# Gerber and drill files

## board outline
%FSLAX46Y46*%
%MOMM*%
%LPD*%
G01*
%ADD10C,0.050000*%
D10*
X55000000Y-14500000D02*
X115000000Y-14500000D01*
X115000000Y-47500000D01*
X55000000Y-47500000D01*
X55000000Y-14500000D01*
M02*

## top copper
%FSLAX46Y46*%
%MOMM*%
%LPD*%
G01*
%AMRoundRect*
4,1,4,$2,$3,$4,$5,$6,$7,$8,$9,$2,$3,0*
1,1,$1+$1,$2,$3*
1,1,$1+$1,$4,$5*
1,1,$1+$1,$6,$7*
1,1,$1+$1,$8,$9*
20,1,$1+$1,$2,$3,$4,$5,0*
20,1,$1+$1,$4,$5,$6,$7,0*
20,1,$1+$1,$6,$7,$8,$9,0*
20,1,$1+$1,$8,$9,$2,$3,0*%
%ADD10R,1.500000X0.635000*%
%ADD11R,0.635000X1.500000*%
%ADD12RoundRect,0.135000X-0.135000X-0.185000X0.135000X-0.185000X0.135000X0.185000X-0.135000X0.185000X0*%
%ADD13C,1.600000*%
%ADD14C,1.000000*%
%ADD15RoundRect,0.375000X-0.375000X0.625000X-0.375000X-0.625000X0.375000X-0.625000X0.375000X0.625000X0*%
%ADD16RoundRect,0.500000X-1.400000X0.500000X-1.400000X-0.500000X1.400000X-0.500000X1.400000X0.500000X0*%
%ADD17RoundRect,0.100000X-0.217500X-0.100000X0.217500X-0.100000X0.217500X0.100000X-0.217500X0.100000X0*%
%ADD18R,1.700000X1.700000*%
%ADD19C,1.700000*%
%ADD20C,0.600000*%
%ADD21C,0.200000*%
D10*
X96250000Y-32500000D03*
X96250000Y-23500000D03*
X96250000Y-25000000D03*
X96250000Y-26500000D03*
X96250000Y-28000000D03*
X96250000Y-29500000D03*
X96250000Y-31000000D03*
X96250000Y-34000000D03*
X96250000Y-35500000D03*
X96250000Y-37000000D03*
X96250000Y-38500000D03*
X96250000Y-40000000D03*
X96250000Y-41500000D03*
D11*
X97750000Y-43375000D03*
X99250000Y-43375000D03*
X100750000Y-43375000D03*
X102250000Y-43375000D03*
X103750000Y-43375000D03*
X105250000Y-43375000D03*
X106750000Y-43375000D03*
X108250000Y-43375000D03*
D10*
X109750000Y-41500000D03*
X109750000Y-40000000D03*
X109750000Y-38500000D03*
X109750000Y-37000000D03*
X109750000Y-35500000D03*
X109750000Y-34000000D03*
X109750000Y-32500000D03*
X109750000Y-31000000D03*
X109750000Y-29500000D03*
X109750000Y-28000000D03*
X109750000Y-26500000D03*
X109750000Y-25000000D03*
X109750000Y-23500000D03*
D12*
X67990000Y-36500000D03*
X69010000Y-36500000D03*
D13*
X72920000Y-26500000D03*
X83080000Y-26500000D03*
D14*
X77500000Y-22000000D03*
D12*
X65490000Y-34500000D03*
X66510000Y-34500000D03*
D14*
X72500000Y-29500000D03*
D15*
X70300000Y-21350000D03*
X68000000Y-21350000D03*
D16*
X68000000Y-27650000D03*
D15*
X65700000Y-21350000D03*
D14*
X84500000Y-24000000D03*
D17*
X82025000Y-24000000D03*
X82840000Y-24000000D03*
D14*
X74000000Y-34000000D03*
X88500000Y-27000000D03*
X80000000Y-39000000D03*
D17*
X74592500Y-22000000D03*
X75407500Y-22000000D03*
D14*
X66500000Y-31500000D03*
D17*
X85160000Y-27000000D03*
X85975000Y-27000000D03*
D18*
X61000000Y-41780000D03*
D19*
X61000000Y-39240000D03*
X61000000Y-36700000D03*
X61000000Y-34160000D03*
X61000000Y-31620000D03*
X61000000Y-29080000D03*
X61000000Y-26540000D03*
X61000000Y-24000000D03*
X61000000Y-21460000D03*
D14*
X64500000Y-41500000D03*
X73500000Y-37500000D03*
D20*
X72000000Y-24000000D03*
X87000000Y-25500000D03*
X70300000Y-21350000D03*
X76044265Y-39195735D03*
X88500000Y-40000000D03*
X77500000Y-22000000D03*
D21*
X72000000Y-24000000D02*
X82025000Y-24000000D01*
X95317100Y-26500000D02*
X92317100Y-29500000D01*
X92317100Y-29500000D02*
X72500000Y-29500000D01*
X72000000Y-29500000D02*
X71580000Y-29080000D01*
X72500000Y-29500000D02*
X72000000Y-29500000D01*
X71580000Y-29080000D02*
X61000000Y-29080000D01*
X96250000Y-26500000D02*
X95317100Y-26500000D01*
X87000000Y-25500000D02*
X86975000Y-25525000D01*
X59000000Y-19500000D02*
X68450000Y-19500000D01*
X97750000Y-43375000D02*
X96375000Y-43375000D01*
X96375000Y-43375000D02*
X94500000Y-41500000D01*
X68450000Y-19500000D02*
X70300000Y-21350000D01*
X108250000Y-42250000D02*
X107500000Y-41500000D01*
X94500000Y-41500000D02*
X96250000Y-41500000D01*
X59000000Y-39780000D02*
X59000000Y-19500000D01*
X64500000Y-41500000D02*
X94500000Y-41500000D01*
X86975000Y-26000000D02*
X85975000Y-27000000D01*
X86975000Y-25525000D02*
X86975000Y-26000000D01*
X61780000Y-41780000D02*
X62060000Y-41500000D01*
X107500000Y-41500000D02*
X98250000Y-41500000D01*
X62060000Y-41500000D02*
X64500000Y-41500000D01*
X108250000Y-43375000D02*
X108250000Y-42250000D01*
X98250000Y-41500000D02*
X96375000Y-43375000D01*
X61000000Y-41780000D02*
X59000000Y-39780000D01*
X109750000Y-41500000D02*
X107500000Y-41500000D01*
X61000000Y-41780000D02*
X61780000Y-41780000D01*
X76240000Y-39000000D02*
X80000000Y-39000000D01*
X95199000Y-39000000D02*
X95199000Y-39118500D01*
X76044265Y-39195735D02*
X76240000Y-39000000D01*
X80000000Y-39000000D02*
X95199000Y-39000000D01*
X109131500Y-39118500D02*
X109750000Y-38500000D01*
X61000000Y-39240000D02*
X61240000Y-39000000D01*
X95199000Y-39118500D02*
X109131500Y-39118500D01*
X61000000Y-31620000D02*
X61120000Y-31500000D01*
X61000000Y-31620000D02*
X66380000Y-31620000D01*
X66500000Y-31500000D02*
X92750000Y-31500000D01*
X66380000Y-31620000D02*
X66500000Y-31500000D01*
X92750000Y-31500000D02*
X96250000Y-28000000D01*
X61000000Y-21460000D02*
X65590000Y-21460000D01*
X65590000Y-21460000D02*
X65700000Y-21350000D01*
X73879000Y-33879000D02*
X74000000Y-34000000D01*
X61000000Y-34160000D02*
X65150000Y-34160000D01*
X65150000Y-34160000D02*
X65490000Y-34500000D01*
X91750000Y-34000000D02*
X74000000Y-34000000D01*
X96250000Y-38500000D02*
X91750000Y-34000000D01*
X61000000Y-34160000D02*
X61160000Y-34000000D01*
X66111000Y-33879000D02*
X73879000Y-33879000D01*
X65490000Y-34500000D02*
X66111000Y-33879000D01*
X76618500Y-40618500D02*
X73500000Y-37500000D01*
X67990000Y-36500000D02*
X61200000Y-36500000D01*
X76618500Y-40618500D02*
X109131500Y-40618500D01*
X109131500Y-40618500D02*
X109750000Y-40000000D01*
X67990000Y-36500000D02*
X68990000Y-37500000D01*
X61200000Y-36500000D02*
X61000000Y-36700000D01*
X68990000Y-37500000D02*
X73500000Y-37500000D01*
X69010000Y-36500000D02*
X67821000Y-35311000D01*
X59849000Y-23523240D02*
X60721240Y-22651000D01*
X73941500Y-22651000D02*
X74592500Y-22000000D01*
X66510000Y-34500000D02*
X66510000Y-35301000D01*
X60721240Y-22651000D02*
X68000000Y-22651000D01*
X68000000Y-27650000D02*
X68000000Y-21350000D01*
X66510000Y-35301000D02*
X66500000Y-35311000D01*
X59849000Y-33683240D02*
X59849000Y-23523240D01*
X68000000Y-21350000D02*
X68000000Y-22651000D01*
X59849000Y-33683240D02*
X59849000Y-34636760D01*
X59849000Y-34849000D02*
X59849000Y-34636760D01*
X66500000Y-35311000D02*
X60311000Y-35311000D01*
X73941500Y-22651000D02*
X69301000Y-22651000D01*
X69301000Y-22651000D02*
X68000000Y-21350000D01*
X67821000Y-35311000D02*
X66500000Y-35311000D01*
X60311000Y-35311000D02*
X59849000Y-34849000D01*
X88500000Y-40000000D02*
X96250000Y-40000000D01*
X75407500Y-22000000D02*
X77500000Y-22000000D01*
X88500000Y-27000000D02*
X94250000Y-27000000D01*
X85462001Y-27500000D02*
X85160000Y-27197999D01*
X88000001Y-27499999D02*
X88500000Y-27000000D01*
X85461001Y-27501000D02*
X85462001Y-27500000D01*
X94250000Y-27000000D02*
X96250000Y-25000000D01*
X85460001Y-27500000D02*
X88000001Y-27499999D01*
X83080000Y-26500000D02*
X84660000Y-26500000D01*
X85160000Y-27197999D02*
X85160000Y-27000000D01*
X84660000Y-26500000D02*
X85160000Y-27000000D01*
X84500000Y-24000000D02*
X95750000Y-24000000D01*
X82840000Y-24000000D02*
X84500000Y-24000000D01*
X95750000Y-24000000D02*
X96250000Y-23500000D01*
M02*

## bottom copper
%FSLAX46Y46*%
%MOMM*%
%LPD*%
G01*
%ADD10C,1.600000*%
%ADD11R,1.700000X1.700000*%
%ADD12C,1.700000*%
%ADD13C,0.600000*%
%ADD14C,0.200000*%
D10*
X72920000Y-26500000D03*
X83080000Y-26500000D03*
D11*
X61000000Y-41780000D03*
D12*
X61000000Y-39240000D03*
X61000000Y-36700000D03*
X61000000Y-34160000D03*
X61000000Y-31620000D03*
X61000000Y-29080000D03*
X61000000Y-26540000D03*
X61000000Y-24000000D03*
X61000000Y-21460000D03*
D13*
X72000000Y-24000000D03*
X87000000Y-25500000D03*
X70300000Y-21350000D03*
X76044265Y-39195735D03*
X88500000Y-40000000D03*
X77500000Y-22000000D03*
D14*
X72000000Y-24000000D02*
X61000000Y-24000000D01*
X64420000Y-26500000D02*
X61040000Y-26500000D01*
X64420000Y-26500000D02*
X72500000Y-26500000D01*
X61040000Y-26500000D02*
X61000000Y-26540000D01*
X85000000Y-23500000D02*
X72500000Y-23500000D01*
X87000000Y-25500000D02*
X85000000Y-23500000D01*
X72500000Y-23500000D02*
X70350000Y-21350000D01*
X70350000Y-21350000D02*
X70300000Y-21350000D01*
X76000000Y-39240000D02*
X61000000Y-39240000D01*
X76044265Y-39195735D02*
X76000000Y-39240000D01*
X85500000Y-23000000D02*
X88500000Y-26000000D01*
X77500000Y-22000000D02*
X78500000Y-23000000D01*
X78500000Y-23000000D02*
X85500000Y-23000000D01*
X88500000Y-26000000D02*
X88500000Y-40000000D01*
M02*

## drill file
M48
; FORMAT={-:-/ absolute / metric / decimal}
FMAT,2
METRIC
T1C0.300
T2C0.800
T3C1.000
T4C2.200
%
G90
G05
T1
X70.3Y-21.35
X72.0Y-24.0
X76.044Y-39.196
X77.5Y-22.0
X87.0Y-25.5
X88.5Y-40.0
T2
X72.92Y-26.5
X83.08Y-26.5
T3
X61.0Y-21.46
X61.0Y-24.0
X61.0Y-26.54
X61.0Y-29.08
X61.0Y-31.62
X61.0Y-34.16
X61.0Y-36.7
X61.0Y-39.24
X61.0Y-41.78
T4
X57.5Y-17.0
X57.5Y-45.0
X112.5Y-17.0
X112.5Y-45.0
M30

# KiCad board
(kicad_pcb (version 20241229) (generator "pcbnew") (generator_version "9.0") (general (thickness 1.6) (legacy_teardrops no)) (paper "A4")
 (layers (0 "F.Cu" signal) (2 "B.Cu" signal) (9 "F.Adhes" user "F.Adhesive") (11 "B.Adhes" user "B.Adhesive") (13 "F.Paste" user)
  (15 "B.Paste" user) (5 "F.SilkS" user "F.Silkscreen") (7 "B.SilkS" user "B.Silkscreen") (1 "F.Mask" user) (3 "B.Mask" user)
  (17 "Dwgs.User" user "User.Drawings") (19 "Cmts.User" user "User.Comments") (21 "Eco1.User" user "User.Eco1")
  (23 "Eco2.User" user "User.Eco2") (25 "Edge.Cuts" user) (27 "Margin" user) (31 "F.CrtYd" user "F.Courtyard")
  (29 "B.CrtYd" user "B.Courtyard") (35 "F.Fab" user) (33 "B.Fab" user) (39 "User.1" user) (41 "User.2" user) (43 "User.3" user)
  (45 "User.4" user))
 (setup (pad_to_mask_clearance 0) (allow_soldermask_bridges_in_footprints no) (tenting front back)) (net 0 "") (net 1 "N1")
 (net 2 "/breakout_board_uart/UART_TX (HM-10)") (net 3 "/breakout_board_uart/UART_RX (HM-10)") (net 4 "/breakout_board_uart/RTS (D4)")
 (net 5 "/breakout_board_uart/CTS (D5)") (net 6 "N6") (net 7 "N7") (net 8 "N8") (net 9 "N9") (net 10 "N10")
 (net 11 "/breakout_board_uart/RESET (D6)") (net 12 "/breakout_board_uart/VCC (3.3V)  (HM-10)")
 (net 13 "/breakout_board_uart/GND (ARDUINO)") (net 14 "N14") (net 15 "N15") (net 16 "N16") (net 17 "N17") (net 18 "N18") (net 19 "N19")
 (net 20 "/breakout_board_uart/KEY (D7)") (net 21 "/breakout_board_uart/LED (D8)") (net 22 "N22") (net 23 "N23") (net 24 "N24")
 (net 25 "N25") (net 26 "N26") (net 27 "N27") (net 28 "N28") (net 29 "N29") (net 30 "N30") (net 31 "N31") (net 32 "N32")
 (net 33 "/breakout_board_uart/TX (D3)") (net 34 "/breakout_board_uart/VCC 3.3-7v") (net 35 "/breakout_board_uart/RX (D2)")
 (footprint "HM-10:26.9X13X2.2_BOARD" (layer "F.Cu") (at 103.75 23.5)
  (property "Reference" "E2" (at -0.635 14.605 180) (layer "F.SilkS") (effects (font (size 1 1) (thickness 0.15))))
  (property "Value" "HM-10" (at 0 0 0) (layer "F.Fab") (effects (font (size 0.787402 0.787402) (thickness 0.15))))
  (pad "$7" smd rect (at -7.5 9) (size 1.5 0.635) (layers "F.Cu" "F.Mask" "F.Paste") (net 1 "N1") (solder_mask_margin 0.102))
  (pad "1" smd rect (at -7.5 0) (size 1.5 0.635) (layers "F.Cu" "F.Mask" "F.Paste") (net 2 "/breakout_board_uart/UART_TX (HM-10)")
   (solder_mask_margin 0.102))
  (pad "2" smd rect (at -7.5 1.5) (size 1.5 0.635) (layers "F.Cu" "F.Mask" "F.Paste") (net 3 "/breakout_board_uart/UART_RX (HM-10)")
   (solder_mask_margin 0.102))
  (pad "3" smd rect (at -7.5 3) (size 1.5 0.635) (layers "F.Cu" "F.Mask" "F.Paste") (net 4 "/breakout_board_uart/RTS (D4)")
   (solder_mask_margin 0.102))
  (pad "4" smd rect (at -7.5 4.5) (size 1.5 0.635) (layers "F.Cu" "F.Mask" "F.Paste") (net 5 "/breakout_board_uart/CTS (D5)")
   (solder_mask_margin 0.102))
  (pad "5" smd rect (at -7.5 6) (size 1.5 0.635) (layers "F.Cu" "F.Mask" "F.Paste") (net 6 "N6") (solder_mask_margin 0.102))
  (pad "6" smd rect (at -7.5 7.5) (size 1.5 0.635) (layers "F.Cu" "F.Mask" "F.Paste") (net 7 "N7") (solder_mask_margin 0.102))
  (pad "8" smd rect (at -7.5 10.5) (size 1.5 0.635) (layers "F.Cu" "F.Mask" "F.Paste") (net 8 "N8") (solder_mask_margin 0.102))
  (pad "9" smd rect (at -7.5 12) (size 1.5 0.635) (layers "F.Cu" "F.Mask" "F.Paste") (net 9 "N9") (solder_mask_margin 0.102))
  (pad "10" smd rect (at -7.5 13.5) (size 1.5 0.635) (layers "F.Cu" "F.Mask" "F.Paste") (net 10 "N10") (solder_mask_margin 0.102))
  (pad "11" smd rect (at -7.5 15) (size 1.5 0.635) (layers "F.Cu" "F.Mask" "F.Paste") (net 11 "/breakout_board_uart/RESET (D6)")
   (solder_mask_margin 0.102))
  (pad "12" smd rect (at -7.5 16.5) (size 1.5 0.635) (layers "F.Cu" "F.Mask" "F.Paste") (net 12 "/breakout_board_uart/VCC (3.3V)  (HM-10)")
   (solder_mask_margin 0.102))
  (pad "13" smd rect (at -7.5 18) (size 1.5 0.635) (layers "F.Cu" "F.Mask" "F.Paste") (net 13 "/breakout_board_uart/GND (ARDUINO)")
   (solder_mask_margin 0.102))
  (pad "14" smd rect (at -6 19.875) (size 0.635 1.5) (layers "F.Cu" "F.Mask" "F.Paste") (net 13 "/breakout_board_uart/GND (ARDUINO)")
   (solder_mask_margin 0.102))
  (pad "15" smd rect (at -4.5 19.875) (size 0.635 1.5) (layers "F.Cu" "F.Mask" "F.Paste") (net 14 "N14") (solder_mask_margin 0.102))
  (pad "16" smd rect (at -3 19.875) (size 0.635 1.5) (layers "F.Cu" "F.Mask" "F.Paste") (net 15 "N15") (solder_mask_margin 0.102))
  (pad "17" smd rect (at -1.5 19.875) (size 0.635 1.5) (layers "F.Cu" "F.Mask" "F.Paste") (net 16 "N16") (solder_mask_margin 0.102))
  (pad "18" smd rect (at 0 19.875) (size 0.635 1.5) (layers "F.Cu" "F.Mask" "F.Paste") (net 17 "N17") (solder_mask_margin 0.102))
  (pad "19" smd rect (at 1.5 19.875) (size 0.635 1.5) (layers "F.Cu" "F.Mask" "F.Paste") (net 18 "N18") (solder_mask_margin 0.102))
  (pad "20" smd rect (at 3 19.875) (size 0.635 1.5) (layers "F.Cu" "F.Mask" "F.Paste") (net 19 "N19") (solder_mask_margin 0.102))
  (pad "21" smd rect (at 4.5 19.875) (size 0.635 1.5) (layers "F.Cu" "F.Mask" "F.Paste") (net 13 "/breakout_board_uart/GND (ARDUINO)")
   (solder_mask_margin 0.102))
  (pad "22" smd rect (at 6 18) (size 1.5 0.635) (layers "F.Cu" "F.Mask" "F.Paste") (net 13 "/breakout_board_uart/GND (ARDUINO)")
   (solder_mask_margin 0.102))
  (pad "23" smd rect (at 6 16.5) (size 1.5 0.635) (layers "F.Cu" "F.Mask" "F.Paste") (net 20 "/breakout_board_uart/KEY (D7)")
   (solder_mask_margin 0.102))
  (pad "24" smd rect (at 6 15) (size 1.5 0.635) (layers "F.Cu" "F.Mask" "F.Paste") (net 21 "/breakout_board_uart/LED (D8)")
   (solder_mask_margin 0.102))
  (pad "25" smd rect (at 6 13.5) (size 1.5 0.635) (layers "F.Cu" "F.Mask" "F.Paste") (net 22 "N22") (solder_mask_margin 0.102))
  (pad "26" smd rect (at 6 12) (size 1.5 0.635) (layers "F.Cu" "F.Mask" "F.Paste") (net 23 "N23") (solder_mask_margin 0.102))
  (pad "27" smd rect (at 6 10.5) (size 1.5 0.635) (layers "F.Cu" "F.Mask" "F.Paste") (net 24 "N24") (solder_mask_margin 0.102))
  (pad "28" smd rect (at 6 9) (size 1.5 0.635) (layers "F.Cu" "F.Mask" "F.Paste") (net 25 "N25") (solder_mask_margin 0.102))
  (pad "29" smd rect (at 6 7.5) (size 1.5 0.635) (layers "F.Cu" "F.Mask" "F.Paste") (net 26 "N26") (solder_mask_margin 0.102))
  (pad "30" smd rect (at 6 6) (size 1.5 0.635) (layers "F.Cu" "F.Mask" "F.Paste") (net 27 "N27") (solder_mask_margin 0.102))
  (pad "31" smd rect (at 6 4.5) (size 1.5 0.635) (layers "F.Cu" "F.Mask" "F.Paste") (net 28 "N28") (solder_mask_margin 0.102))
  (pad "32" smd rect (at 6 3) (size 1.5 0.635) (layers "F.Cu" "F.Mask" "F.Paste") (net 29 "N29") (solder_mask_margin 0.102))
  (pad "33" smd rect (at 6 1.5) (size 1.5 0.635) (layers "F.Cu" "F.Mask" "F.Paste") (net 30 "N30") (solder_mask_margin 0.102))
  (pad "34" smd rect (at 6 0) (size 1.5 0.635) (layers "F.Cu" "F.Mask" "F.Paste") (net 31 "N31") (solder_mask_margin 0.102)))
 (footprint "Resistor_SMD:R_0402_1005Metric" (layer "F.Cu") (at 68.5 36.5)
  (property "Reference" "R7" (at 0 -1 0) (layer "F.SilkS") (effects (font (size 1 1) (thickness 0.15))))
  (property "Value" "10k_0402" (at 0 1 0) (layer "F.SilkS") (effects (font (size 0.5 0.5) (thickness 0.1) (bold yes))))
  (pad "1" smd roundrect (at -0.51 0) (size 0.54 0.64) (layers "F.Cu" "F.Mask" "F.Paste") (roundrect_rratio 0.25)
   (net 20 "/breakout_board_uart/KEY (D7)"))
  (pad "2" smd roundrect (at 0.51 0) (size 0.54 0.64) (layers "F.Cu" "F.Mask" "F.Paste") (roundrect_rratio 0.25) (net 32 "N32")))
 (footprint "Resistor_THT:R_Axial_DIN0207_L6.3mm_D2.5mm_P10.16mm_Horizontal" (layer "F.Cu") (at 72.92 26.5)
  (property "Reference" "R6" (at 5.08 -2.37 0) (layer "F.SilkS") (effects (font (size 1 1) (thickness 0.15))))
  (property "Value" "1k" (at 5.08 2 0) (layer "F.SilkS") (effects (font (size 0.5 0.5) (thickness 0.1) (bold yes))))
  (pad "1" thru_hole circle (at 0 0) (size 1.6 1.6) (drill 0.8) (layers "*.Cu" "*.Mask") (remove_unused_layers no)
   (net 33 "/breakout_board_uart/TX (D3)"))
  (pad "2" thru_hole circle (at 10.16 0) (size 1.6 1.6) (drill 0.8) (layers "*.Cu" "*.Mask") (remove_unused_layers no)
   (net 3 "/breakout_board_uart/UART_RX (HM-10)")))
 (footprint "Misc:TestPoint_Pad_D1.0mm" (layer "F.Cu") (at 77.5 22)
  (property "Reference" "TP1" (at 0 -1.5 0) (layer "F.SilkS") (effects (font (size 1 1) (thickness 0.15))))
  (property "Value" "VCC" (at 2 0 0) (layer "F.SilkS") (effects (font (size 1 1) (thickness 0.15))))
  (pad "1" smd circle (at 0 0) (size 1 1) (layers "F.Cu" "F.Mask") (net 12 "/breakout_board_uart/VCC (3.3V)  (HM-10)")))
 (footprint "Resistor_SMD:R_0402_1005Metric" (layer "F.Cu") (at 66 34.5)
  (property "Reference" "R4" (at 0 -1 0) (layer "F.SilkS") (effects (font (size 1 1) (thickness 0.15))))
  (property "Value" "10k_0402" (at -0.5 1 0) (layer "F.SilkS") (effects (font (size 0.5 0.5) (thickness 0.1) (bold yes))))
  (pad "1" smd roundrect (at -0.51 0) (size 0.54 0.64) (layers "F.Cu" "F.Mask" "F.Paste") (roundrect_rratio 0.25)
   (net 11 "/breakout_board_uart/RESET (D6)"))
  (pad "2" smd roundrect (at 0.51 0) (size 0.54 0.64) (layers "F.Cu" "F.Mask" "F.Paste") (roundrect_rratio 0.25) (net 32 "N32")))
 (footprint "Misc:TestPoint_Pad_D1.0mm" (layer "F.Cu") (at 72.5 29.5)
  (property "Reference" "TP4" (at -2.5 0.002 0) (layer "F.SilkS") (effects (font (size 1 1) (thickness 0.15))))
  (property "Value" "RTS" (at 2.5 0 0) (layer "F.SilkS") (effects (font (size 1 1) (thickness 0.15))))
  (pad "1" smd circle (at 0 0) (size 1 1) (layers "F.Cu" "F.Mask") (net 4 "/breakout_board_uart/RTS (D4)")))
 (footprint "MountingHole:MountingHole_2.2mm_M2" (layer "F.Cu") (at 112.5 45)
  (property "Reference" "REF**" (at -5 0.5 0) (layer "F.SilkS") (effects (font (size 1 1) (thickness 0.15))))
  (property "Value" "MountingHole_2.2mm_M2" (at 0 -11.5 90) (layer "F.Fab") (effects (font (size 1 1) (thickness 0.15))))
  (pad "" np_thru_hole circle (at 0 0) (size 2.2 2.2) (drill 2.2) (layers "*.Cu" "*.Mask")))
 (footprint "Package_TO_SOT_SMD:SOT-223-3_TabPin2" (layer "F.Cu") (at 68 24.5 -90)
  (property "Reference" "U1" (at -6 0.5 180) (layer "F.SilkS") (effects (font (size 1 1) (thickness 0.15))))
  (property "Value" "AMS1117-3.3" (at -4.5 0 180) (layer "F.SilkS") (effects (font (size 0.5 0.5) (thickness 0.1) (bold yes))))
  (pad "1" smd roundrect (at -3.15 -2.3 270) (size 2 1.5) (layers "F.Cu" "F.Mask" "F.Paste") (roundrect_rratio 0.25)
   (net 13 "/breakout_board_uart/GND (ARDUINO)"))
  (pad "2" smd roundrect (at -3.15 0 270) (size 2 1.5) (layers "F.Cu" "F.Mask" "F.Paste") (roundrect_rratio 0.25) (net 32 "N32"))
  (pad "2" smd roundrect (at 3.15 0 270) (size 2 3.8) (layers "F.Cu" "F.Mask" "F.Paste") (roundrect_rratio 0.25) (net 32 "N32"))
  (pad "3" smd roundrect (at -3.15 2.3 270) (size 2 1.5) (layers "F.Cu" "F.Mask" "F.Paste") (roundrect_rratio 0.25)
   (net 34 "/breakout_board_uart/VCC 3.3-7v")))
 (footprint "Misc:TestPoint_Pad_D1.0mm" (layer "F.Cu") (at 84.5 24)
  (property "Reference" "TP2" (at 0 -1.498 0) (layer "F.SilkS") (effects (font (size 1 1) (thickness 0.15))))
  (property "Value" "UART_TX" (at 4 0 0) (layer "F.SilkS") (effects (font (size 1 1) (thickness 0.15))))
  (pad "1" smd circle (at 0 0) (size 1 1) (layers "F.Cu" "F.Mask") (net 2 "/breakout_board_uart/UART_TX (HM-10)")))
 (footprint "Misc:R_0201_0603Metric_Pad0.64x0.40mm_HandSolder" (layer "F.Cu") (at 82.4325 24)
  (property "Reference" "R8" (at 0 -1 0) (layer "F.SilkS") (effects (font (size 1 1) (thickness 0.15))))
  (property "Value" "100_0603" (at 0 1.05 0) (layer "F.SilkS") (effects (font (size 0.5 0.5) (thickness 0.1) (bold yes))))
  (pad "" smd roundrect (at -0.4325 0) (size 0.458 0.36) (layers "F.Paste") (roundrect_rratio 0.25))
  (pad "" smd roundrect (at 0.4325 0) (size 0.458 0.36) (layers "F.Paste") (roundrect_rratio 0.25))
  (pad "1" smd roundrect (at -0.4075 0) (size 0.635 0.4) (layers "F.Cu" "F.Mask") (roundrect_rratio 0.25)
   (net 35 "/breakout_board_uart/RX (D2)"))
  (pad "2" smd roundrect (at 0.4075 0) (size 0.635 0.4) (layers "F.Cu" "F.Mask") (roundrect_rratio 0.25)
   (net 2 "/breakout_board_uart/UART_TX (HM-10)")))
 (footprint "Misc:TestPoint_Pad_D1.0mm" (layer "F.Cu") (at 74 34)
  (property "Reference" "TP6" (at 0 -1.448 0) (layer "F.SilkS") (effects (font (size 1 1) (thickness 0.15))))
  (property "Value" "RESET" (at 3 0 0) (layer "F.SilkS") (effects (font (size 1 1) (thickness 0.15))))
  (pad "1" smd circle (at 0 0) (size 1 1) (layers "F.Cu" "F.Mask") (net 11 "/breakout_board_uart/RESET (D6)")))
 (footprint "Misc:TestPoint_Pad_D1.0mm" (layer "F.Cu") (at 88.5 27)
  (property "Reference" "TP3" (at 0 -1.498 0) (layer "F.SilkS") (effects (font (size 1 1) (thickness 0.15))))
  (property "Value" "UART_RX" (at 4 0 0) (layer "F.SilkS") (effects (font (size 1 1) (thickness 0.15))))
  (pad "1" smd circle (at 0 0) (size 1 1) (layers "F.Cu" "F.Mask") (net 3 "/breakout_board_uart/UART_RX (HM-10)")))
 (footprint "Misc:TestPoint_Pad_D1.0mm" (layer "F.Cu") (at 80 39)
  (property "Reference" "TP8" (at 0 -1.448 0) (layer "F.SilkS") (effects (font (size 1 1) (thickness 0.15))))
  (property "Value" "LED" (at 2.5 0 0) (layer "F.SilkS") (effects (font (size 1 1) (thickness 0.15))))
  (pad "1" smd circle (at 0 0) (size 1 1) (layers "F.Cu" "F.Mask") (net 21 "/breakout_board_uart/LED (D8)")))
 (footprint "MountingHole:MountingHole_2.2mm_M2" (layer "F.Cu") (at 57.5 45)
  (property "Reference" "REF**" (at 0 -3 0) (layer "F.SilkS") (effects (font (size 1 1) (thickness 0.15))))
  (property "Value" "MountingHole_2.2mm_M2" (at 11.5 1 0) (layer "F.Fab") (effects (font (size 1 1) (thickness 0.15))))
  (pad "" np_thru_hole circle (at 0 0) (size 2.2 2.2) (drill 2.2) (layers "*.Cu" "*.Mask")))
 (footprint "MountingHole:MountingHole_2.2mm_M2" (layer "F.Cu") (at 112.5 17)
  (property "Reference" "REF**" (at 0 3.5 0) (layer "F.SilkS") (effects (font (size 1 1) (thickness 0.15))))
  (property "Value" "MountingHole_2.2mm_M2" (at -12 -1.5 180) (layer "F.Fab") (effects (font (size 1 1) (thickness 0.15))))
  (pad "" np_thru_hole circle (at 0 0) (size 2.2 2.2) (drill 2.2) (layers "*.Cu" "*.Mask")))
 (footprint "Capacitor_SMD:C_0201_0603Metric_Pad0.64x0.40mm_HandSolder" (layer "F.Cu") (at 75 22)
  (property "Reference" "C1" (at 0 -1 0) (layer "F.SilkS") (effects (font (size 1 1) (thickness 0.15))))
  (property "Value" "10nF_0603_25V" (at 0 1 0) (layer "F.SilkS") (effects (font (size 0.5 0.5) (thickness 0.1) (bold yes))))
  (pad "" smd roundrect (at -0.4325 0) (size 0.458 0.36) (layers "F.Paste") (roundrect_rratio 0.25))
  (pad "" smd roundrect (at 0.4325 0) (size 0.458 0.36) (layers "F.Paste") (roundrect_rratio 0.25))
  (pad "1" smd roundrect (at -0.4075 0) (size 0.635 0.4) (layers "F.Cu" "F.Mask") (roundrect_rratio 0.25) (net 32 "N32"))
  (pad "2" smd roundrect (at 0.4075 0) (size 0.635 0.4) (layers "F.Cu" "F.Mask") (roundrect_rratio 0.25)
   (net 12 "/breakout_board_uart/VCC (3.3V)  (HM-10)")))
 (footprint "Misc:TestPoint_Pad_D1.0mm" (layer "F.Cu") (at 66.5 31.5)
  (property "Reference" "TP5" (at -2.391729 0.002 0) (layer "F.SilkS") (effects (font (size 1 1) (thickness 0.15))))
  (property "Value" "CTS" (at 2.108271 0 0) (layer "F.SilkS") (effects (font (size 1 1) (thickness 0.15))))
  (pad "1" smd circle (at 0 0) (size 1 1) (layers "F.Cu" "F.Mask") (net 5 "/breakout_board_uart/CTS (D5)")))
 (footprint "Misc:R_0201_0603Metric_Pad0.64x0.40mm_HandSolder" (layer "F.Cu") (at 85.5675 27)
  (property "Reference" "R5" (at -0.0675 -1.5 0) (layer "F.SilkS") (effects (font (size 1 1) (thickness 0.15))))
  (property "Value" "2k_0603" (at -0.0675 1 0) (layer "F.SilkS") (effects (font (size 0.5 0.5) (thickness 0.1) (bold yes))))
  (pad "" smd roundrect (at -0.4325 0) (size 0.458 0.36) (layers "F.Paste") (roundrect_rratio 0.25))
  (pad "" smd roundrect (at 0.4325 0) (size 0.458 0.36) (layers "F.Paste") (roundrect_rratio 0.25))
  (pad "1" smd roundrect (at -0.4075 0) (size 0.635 0.4) (layers "F.Cu" "F.Mask") (roundrect_rratio 0.25)
   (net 3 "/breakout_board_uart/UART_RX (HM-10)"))
  (pad "2" smd roundrect (at 0.4075 0) (size 0.635 0.4) (layers "F.Cu" "F.Mask") (roundrect_rratio 0.25)
   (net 13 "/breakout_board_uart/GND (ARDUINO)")))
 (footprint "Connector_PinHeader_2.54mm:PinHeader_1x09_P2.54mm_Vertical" (layer "F.Cu") (at 61 41.78 180)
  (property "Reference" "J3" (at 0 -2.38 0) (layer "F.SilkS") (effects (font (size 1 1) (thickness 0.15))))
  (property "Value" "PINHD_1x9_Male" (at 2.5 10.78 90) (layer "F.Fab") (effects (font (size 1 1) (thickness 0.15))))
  (pad "1" thru_hole rect (at 0 0 180) (size 1.7 1.7) (drill 1) (layers "*.Cu" "*.Mask") (remove_unused_layers no)
   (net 13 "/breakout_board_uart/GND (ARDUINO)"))
  (pad "2" thru_hole circle (at 0 2.54 180) (size 1.7 1.7) (drill 1) (layers "*.Cu" "*.Mask") (remove_unused_layers no)
   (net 21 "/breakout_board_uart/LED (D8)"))
  (pad "3" thru_hole circle (at 0 5.08 180) (size 1.7 1.7) (drill 1) (layers "*.Cu" "*.Mask") (remove_unused_layers no)
   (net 20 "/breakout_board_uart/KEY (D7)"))
  (pad "4" thru_hole circle (at 0 7.62 180) (size 1.7 1.7) (drill 1) (layers "*.Cu" "*.Mask") (remove_unused_layers no)
   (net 11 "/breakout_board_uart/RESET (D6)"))
  (pad "5" thru_hole circle (at 0 10.16 180) (size 1.7 1.7) (drill 1) (layers "*.Cu" "*.Mask") (remove_unused_layers no)
   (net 5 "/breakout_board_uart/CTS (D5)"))
  (pad "6" thru_hole circle (at 0 12.7 180) (size 1.7 1.7) (drill 1) (layers "*.Cu" "*.Mask") (remove_unused_layers no)
   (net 4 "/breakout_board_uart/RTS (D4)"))
  (pad "7" thru_hole circle (at 0 15.24 180) (size 1.7 1.7) (drill 1) (layers "*.Cu" "*.Mask") (remove_unused_layers no)
   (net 33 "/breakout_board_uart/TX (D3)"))
  (pad "8" thru_hole circle (at 0 17.78 180) (size 1.7 1.7) (drill 1) (layers "*.Cu" "*.Mask") (remove_unused_layers no)
   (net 35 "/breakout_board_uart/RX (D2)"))
  (pad "9" thru_hole circle (at 0 20.32 180) (size 1.7 1.7) (drill 1) (layers "*.Cu" "*.Mask") (remove_unused_layers no)
   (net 34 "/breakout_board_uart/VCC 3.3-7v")))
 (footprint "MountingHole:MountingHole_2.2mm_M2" (layer "F.Cu") (at 57.5 17)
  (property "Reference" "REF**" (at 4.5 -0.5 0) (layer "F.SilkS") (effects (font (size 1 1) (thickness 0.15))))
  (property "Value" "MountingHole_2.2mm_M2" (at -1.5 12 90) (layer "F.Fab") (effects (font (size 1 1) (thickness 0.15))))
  (pad "" np_thru_hole circle (at 0 0) (size 2.2 2.2) (drill 2.2) (layers "*.Cu" "*.Mask")))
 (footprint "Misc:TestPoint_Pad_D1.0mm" (layer "F.Cu") (at 64.5 41.5)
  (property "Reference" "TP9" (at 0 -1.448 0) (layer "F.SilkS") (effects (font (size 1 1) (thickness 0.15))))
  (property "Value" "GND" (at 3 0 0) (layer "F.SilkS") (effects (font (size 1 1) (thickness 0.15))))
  (pad "1" smd circle (at 0 0) (size 1 1) (layers "F.Cu" "F.Mask") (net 13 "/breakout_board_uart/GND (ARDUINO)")))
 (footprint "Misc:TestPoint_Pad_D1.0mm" (layer "F.Cu") (at 73.5 37.5)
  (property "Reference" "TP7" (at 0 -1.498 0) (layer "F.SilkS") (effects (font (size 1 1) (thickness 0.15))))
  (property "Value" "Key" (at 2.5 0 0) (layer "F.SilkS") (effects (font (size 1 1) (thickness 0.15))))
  (pad "1" smd circle (at 0 0) (size 1 1) (layers "F.Cu" "F.Mask") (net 20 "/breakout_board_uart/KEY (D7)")))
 (gr_rect (start 55 14.5) (end 115 47.5) (stroke (width 0.05) (type default)) (fill no) (layer "Edge.Cuts"))
 (segment (start 72 24) (end 82.025 24) (width 0.2) (layer "F.Cu") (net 35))
 (via (at 72 24) (size 0.6) (drill 0.3) (layers "F.Cu" "B.Cu") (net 35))
 (segment (start 72 24) (end 61 24) (width 0.2) (layer "B.Cu") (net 35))
 (segment (start 95.3171 26.5) (end 92.3171 29.5) (width 0.2) (layer "F.Cu") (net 4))
 (segment (start 92.3171 29.5) (end 72.5 29.5) (width 0.2) (layer "F.Cu") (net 4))
 (segment (start 72 29.5) (end 71.58 29.08) (width 0.2) (layer "F.Cu") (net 4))
 (segment (start 72.5 29.5) (end 72 29.5) (width 0.2) (layer "F.Cu") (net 4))
 (segment (start 71.58 29.08) (end 61 29.08) (width 0.2) (layer "F.Cu") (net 4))
 (segment (start 96.25 26.5) (end 95.3171 26.5) (width 0.2) (layer "F.Cu") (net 4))
 (segment (start 64.42 26.5) (end 61.04 26.5) (width 0.2) (layer "B.Cu") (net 33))
 (segment (start 64.42 26.5) (end 72.5 26.5) (width 0.2) (layer "B.Cu") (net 33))
 (segment (start 61.04 26.5) (end 61 26.54) (width 0.2) (layer "B.Cu") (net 33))
 (segment (start 87 25.5) (end 86.975 25.525) (width 0.2) (layer "F.Cu") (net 13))
 (segment (start 59 19.5) (end 68.45 19.5) (width 0.2) (layer "F.Cu") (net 13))
 (segment (start 97.75 43.375) (end 96.375 43.375) (width 0.2) (layer "F.Cu") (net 13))
 (segment (start 96.375 43.375) (end 94.5 41.5) (width 0.2) (layer "F.Cu") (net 13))
 (segment (start 68.45 19.5) (end 70.3 21.35) (width 0.2) (layer "F.Cu") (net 13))
 (segment (start 108.25 42.25) (end 107.5 41.5) (width 0.2) (layer "F.Cu") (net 13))
 (segment (start 94.5 41.5) (end 96.25 41.5) (width 0.2) (layer "F.Cu") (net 13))
 (segment (start 59 39.78) (end 59 19.5) (width 0.2) (layer "F.Cu") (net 13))
 (segment (start 64.5 41.5) (end 94.5 41.5) (width 0.2) (layer "F.Cu") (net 13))
 (segment (start 86.975 26) (end 85.975 27) (width 0.2) (layer "F.Cu") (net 13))
 (segment (start 86.975 25.525) (end 86.975 26) (width 0.2) (layer "F.Cu") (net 13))
 (segment (start 61.78 41.78) (end 62.06 41.5) (width 0.2) (layer "F.Cu") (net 13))
 (segment (start 107.5 41.5) (end 98.25 41.5) (width 0.2) (layer "F.Cu") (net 13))
 (segment (start 62.06 41.5) (end 64.5 41.5) (width 0.2) (layer "F.Cu") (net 13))
 (segment (start 108.25 43.375) (end 108.25 42.25) (width 0.2) (layer "F.Cu") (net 13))
 (segment (start 98.25 41.5) (end 96.375 43.375) (width 0.2) (layer "F.Cu") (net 13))
 (segment (start 61 41.78) (end 59 39.78) (width 0.2) (layer "F.Cu") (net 13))
 (segment (start 109.75 41.5) (end 107.5 41.5) (width 0.2) (layer "F.Cu") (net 13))
 (segment (start 61 41.78) (end 61.78 41.78) (width 0.2) (layer "F.Cu") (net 13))
 (via (at 87 25.5) (size 0.6) (drill 0.3) (layers "F.Cu" "B.Cu") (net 13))
 (via (at 70.3 21.35) (size 0.6) (drill 0.3) (layers "F.Cu" "B.Cu") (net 13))
 (segment (start 85 23.5) (end 72.5 23.5) (width 0.2) (layer "B.Cu") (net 13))
 (segment (start 87 25.5) (end 85 23.5) (width 0.2) (layer "B.Cu") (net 13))
 (segment (start 72.5 23.5) (end 70.35 21.35) (width 0.2) (layer "B.Cu") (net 13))
 (segment (start 70.35 21.35) (end 70.3 21.35) (width 0.2) (layer "B.Cu") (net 13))
 (segment (start 76.24 39) (end 80 39) (width 0.2) (layer "F.Cu") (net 21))
 (segment (start 95.199 39) (end 95.199 39.1185) (width 0.2) (layer "F.Cu") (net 21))
 (segment (start 76.044265 39.195735) (end 76.24 39) (width 0.2) (layer "F.Cu") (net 21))
 (segment (start 80 39) (end 95.199 39) (width 0.2) (layer "F.Cu") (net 21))
 (segment (start 109.1315 39.1185) (end 109.75 38.5) (width 0.2) (layer "F.Cu") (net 21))
 (segment (start 61 39.24) (end 61.24 39) (width 0.2) (layer "F.Cu") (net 21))
 (segment (start 95.199 39.1185) (end 109.1315 39.1185) (width 0.2) (layer "F.Cu") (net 21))
 (via (at 76.044265 39.195735) (size 0.6) (drill 0.3) (layers "F.Cu" "B.Cu") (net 21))
 (segment (start 76 39.24) (end 61 39.24) (width 0.2) (layer "B.Cu") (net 21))
 (segment (start 76.044265 39.195735) (end 76 39.24) (width 0.2) (layer "B.Cu") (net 21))
 (segment (start 61 31.62) (end 61.12 31.5) (width 0.2) (layer "F.Cu") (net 5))
 (segment (start 61 31.62) (end 66.38 31.62) (width 0.2) (layer "F.Cu") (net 5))
 (segment (start 66.5 31.5) (end 92.75 31.5) (width 0.2) (layer "F.Cu") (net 5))
 (segment (start 66.38 31.62) (end 66.5 31.5) (width 0.2) (layer "F.Cu") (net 5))
 (segment (start 92.75 31.5) (end 96.25 28) (width 0.2) (layer "F.Cu") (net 5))
 (segment (start 61 21.46) (end 65.59 21.46) (width 0.2) (layer "F.Cu") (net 34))
 (segment (start 65.59 21.46) (end 65.7 21.35) (width 0.2) (layer "F.Cu") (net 34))
 (segment (start 73.879 33.879) (end 74 34) (width 0.2) (layer "F.Cu") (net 11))
 (segment (start 61 34.16) (end 65.15 34.16) (width 0.2) (layer "F.Cu") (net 11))
 (segment (start 65.15 34.16) (end 65.49 34.5) (width 0.2) (layer "F.Cu") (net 11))
 (segment (start 91.75 34) (end 74 34) (width 0.2) (layer "F.Cu") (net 11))
 (segment (start 96.25 38.5) (end 91.75 34) (width 0.2) (layer "F.Cu") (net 11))
 (segment (start 61 34.16) (end 61.16 34) (width 0.2) (layer "F.Cu") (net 11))
 (segment (start 66.111 33.879) (end 73.879 33.879) (width 0.2) (layer "F.Cu") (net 11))
 (segment (start 65.49 34.5) (end 66.111 33.879) (width 0.2) (layer "F.Cu") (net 11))
 (segment (start 76.6185 40.6185) (end 73.5 37.5) (width 0.2) (layer "F.Cu") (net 20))
 (segment (start 67.99 36.5) (end 61.2 36.5) (width 0.2) (layer "F.Cu") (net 20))
 (segment (start 76.6185 40.6185) (end 109.1315 40.6185) (width 0.2) (layer "F.Cu") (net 20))
 (segment (start 109.1315 40.6185) (end 109.75 40) (width 0.2) (layer "F.Cu") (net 20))
 (segment (start 67.99 36.5) (end 68.99 37.5) (width 0.2) (layer "F.Cu") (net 20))
 (segment (start 61.2 36.5) (end 61 36.7) (width 0.2) (layer "F.Cu") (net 20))
 (segment (start 68.99 37.5) (end 73.5 37.5) (width 0.2) (layer "F.Cu") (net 20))
 (segment (start 69.01 36.5) (end 67.821 35.311) (width 0.2) (layer "F.Cu") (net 32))
 (segment (start 59.849 23.52324) (end 60.72124 22.651) (width 0.2) (layer "F.Cu") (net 32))
 (segment (start 73.9415 22.651) (end 74.5925 22) (width 0.2) (layer "F.Cu") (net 32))
 (segment (start 66.51 34.5) (end 66.51 35.301) (width 0.2) (layer "F.Cu") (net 32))
 (segment (start 60.72124 22.651) (end 68 22.651) (width 0.2) (layer "F.Cu") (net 32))
 (segment (start 68 27.65) (end 68 21.35) (width 0.2) (layer "F.Cu") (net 32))
 (segment (start 66.51 35.301) (end 66.5 35.311) (width 0.2) (layer "F.Cu") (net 32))
 (segment (start 59.849 33.68324) (end 59.849 23.52324) (width 0.2) (layer "F.Cu") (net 32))
 (segment (start 68 21.35) (end 68 22.651) (width 0.2) (layer "F.Cu") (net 32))
 (segment (start 59.849 33.68324) (end 59.849 34.63676) (width 0.2) (layer "F.Cu") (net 32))
 (segment (start 59.849 34.849) (end 59.849 34.63676) (width 0.2) (layer "F.Cu") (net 32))
 (segment (start 66.5 35.311) (end 60.311 35.311) (width 0.2) (layer "F.Cu") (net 32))
 (segment (start 73.9415 22.651) (end 69.301 22.651) (width 0.2) (layer "F.Cu") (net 32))
 (segment (start 69.301 22.651) (end 68 21.35) (width 0.2) (layer "F.Cu") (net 32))
 (segment (start 67.821 35.311) (end 66.5 35.311) (width 0.2) (layer "F.Cu") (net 32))
 (segment (start 60.311 35.311) (end 59.849 34.849) (width 0.2) (layer "F.Cu") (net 32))
 (segment (start 88.5 40) (end 96.25 40) (width 0.2) (layer "F.Cu") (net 12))
 (segment (start 75.4075 22) (end 77.5 22) (width 0.2) (layer "F.Cu") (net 12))
 (via (at 88.5 40) (size 0.6) (drill 0.3) (layers "F.Cu" "B.Cu") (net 12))
 (via (at 77.5 22) (size 0.6) (drill 0.3) (layers "F.Cu" "B.Cu") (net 12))
 (segment (start 85.5 23) (end 88.5 26) (width 0.2) (layer "B.Cu") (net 12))
 (segment (start 77.5 22) (end 78.5 23) (width 0.2) (layer "B.Cu") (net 12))
 (segment (start 78.5 23) (end 85.5 23) (width 0.2) (layer "B.Cu") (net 12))
 (segment (start 88.5 26) (end 88.5 40) (width 0.2) (layer "B.Cu") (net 12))
 (segment (start 88.5 27) (end 94.25 27) (width 0.2) (layer "F.Cu") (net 3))
 (segment (start 85.462001 27.5) (end 85.16 27.197999) (width 0.2) (layer "F.Cu") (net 3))
 (segment (start 88.000001 27.499999) (end 88.5 27) (width 0.2) (layer "F.Cu") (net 3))
 (segment (start 85.461001 27.501) (end 85.462001 27.5) (width 0.2) (layer "F.Cu") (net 3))
 (segment (start 94.25 27) (end 96.25 25) (width 0.2) (layer "F.Cu") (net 3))
 (segment (start 85.460001 27.5) (end 88.000001 27.499999) (width 0.2) (layer "F.Cu") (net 3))
 (segment (start 83.08 26.5) (end 84.66 26.5) (width 0.2) (layer "F.Cu") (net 3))
 (segment (start 85.16 27.197999) (end 85.16 27) (width 0.2) (layer "F.Cu") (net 3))
 (segment (start 84.66 26.5) (end 85.16 27) (width 0.2) (layer "F.Cu") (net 3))
 (segment (start 84.5 24) (end 95.75 24) (width 0.2) (layer "F.Cu") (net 2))
 (segment (start 82.84 24) (end 84.5 24) (width 0.2) (layer "F.Cu") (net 2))
 (segment (start 95.75 24) (end 96.25 23.5) (width 0.2) (layer "F.Cu") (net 2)))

